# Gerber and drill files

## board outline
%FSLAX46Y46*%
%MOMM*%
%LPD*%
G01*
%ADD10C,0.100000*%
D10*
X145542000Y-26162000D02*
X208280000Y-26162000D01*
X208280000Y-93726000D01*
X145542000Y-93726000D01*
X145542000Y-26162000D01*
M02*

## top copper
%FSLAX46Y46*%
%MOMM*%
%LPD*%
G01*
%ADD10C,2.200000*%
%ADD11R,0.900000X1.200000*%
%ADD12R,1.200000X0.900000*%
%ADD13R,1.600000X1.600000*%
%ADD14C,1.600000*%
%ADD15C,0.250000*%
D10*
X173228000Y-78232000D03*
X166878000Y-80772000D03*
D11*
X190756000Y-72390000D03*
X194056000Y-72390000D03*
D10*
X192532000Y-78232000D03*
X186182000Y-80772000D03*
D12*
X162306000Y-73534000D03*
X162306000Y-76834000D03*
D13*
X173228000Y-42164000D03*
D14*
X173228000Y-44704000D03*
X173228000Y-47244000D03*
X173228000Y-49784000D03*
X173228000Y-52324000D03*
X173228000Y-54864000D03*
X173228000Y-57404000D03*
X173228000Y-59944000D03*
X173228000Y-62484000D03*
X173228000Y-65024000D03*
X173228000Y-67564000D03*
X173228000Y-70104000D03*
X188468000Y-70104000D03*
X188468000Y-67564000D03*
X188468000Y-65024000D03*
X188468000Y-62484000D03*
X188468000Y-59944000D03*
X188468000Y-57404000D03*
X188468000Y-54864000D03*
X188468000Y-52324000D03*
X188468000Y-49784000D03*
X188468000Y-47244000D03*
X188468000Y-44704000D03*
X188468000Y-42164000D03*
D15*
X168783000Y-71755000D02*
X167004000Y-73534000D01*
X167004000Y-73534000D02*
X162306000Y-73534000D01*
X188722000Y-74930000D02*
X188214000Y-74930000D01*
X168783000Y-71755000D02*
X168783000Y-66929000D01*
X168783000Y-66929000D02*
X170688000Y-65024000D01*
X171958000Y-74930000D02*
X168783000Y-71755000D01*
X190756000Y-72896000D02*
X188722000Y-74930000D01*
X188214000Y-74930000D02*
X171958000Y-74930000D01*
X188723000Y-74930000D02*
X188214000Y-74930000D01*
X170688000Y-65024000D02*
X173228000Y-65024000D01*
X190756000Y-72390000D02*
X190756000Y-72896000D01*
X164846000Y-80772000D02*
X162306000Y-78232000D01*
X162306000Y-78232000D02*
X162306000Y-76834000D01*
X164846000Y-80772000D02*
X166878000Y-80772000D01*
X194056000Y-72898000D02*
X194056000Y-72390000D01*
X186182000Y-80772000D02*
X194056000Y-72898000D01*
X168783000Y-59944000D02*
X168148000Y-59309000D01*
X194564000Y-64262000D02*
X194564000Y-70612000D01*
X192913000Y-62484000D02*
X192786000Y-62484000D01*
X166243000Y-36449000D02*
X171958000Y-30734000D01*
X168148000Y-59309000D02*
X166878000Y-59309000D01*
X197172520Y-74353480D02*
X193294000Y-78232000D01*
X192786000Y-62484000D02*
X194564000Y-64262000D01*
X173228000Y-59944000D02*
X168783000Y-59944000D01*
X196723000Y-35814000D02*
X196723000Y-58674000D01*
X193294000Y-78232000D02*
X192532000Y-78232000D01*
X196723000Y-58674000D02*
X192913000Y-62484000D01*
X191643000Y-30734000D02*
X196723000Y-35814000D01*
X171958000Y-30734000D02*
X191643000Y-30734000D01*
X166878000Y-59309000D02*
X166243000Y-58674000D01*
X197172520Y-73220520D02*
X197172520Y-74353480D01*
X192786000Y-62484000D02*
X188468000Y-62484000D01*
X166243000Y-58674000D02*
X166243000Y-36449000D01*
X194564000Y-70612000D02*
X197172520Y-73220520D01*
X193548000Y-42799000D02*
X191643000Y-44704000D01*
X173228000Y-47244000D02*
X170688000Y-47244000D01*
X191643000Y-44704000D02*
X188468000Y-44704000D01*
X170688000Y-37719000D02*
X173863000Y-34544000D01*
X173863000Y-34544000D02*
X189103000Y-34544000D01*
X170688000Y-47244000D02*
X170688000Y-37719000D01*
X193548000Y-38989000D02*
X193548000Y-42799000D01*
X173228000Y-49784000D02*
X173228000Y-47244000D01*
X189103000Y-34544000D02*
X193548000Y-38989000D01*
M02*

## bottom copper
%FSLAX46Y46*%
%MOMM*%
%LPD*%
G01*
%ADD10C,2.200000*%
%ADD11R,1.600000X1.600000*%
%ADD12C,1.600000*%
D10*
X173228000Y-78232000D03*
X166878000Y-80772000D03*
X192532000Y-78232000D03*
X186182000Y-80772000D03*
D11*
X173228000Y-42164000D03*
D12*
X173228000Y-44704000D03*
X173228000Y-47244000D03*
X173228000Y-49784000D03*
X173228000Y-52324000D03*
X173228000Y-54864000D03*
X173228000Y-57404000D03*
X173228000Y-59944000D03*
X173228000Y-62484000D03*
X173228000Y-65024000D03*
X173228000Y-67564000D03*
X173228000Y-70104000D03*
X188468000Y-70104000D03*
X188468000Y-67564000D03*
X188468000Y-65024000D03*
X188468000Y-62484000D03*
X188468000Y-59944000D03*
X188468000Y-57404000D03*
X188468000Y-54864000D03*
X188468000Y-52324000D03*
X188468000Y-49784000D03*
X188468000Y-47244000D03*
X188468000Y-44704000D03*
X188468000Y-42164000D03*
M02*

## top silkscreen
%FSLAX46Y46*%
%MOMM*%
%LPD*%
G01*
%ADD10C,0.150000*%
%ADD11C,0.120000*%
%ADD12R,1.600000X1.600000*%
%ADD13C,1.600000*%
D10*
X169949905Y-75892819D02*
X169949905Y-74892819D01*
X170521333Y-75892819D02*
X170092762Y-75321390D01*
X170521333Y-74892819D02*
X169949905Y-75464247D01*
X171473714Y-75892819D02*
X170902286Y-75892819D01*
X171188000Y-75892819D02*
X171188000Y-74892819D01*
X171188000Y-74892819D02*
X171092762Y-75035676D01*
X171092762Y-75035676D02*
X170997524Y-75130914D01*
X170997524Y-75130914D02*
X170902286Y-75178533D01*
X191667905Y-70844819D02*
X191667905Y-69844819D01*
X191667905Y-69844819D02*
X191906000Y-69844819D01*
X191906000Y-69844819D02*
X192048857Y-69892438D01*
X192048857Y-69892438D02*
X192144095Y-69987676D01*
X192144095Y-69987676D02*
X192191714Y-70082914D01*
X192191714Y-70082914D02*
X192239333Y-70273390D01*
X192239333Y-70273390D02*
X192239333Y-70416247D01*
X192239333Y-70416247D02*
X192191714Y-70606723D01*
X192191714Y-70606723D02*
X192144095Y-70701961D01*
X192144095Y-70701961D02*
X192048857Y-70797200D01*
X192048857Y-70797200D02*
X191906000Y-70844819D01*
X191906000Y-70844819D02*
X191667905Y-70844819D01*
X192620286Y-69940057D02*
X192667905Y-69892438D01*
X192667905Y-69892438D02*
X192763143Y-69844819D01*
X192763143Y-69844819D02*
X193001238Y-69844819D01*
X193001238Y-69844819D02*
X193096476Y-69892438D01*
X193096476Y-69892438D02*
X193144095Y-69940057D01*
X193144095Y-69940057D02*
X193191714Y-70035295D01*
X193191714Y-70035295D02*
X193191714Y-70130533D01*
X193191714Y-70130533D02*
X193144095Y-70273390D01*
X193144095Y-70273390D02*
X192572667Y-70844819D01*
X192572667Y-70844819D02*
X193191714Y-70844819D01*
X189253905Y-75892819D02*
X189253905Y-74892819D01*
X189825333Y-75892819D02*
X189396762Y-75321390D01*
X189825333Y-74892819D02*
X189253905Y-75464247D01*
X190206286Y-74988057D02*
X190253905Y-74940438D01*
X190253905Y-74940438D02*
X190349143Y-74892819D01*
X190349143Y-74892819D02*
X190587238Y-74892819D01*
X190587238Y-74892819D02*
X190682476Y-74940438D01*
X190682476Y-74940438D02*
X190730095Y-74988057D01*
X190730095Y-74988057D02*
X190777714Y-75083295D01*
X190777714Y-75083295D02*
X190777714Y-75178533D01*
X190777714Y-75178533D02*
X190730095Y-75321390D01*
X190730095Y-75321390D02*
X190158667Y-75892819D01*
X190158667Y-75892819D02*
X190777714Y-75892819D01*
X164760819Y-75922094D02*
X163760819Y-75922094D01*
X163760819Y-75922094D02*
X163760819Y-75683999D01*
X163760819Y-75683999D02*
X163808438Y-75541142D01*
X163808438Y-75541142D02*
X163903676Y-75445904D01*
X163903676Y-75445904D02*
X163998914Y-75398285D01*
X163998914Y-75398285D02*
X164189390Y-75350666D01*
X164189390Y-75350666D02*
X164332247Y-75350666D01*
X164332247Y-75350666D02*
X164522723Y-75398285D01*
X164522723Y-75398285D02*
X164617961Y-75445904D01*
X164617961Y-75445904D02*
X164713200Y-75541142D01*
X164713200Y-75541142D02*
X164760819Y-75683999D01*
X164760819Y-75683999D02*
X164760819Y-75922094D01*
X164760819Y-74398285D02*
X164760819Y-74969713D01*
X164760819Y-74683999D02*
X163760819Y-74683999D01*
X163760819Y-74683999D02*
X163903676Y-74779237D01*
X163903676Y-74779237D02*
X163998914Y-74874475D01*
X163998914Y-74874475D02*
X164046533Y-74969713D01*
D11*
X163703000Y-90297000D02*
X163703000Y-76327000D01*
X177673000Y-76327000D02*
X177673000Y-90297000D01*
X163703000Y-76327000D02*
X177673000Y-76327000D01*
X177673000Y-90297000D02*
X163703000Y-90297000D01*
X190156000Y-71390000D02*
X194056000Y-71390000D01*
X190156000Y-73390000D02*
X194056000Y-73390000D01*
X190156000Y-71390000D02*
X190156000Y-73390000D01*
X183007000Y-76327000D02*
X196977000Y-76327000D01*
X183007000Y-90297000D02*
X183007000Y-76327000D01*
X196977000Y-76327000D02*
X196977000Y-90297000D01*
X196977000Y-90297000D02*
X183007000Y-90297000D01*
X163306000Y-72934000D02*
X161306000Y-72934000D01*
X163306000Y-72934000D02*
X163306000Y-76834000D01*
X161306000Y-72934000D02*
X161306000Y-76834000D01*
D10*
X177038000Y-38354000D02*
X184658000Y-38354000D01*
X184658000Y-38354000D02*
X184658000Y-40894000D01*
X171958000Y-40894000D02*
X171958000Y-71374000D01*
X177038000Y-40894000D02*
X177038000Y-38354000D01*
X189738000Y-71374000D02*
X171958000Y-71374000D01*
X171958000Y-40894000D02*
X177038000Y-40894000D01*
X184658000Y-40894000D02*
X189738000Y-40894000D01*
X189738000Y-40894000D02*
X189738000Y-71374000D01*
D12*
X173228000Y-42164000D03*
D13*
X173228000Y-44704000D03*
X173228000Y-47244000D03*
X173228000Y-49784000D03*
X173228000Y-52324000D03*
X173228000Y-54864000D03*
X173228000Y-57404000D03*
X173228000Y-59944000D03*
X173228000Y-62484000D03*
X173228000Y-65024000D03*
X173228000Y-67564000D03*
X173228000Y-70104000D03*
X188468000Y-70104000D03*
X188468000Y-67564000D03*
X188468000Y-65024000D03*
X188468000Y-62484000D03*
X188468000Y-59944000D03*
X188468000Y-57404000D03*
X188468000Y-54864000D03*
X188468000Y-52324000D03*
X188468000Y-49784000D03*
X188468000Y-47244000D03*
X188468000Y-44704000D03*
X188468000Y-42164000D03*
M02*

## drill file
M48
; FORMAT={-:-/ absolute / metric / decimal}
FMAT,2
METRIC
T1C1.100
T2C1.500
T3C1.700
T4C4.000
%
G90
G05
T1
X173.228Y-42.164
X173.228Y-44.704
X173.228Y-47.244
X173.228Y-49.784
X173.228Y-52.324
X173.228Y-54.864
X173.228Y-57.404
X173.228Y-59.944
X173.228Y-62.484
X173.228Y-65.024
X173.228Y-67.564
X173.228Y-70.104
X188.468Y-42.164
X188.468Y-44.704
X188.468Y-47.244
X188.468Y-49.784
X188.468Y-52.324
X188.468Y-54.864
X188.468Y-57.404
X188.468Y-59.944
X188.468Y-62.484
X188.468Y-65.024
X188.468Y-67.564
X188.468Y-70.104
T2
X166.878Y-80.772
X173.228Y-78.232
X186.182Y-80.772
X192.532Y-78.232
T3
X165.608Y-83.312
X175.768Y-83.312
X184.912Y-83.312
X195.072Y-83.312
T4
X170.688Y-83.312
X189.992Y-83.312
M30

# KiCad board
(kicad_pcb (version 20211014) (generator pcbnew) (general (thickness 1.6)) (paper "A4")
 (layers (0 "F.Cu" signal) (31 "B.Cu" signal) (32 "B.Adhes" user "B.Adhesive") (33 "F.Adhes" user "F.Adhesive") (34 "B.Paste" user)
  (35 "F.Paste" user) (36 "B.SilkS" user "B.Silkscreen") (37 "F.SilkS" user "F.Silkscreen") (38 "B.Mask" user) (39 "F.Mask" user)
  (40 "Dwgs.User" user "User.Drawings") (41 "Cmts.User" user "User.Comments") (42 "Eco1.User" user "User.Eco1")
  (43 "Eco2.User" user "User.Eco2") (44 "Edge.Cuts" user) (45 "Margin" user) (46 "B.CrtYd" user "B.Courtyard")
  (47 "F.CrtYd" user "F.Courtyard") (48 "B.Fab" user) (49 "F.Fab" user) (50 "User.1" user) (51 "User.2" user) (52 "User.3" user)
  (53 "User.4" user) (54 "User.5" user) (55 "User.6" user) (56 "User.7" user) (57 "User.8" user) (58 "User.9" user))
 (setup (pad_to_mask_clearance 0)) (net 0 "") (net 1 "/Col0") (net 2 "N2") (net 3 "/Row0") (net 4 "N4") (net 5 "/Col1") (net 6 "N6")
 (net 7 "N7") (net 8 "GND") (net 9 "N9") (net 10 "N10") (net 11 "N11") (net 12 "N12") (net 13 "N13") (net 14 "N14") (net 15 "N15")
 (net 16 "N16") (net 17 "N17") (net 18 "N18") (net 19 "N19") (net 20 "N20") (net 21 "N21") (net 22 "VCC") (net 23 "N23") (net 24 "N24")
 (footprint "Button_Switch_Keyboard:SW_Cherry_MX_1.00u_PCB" (layer "F.Cu") (at 173.228 78.232)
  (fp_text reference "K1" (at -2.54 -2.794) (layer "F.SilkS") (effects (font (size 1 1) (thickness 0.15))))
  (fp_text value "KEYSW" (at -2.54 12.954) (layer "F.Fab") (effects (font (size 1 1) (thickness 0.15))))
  (fp_line (start -9.525 12.065) (end -9.525 -1.905) (layer "F.SilkS") (width 0.12))
  (fp_line (start 4.445 -1.905) (end 4.445 12.065) (layer "F.SilkS") (width 0.12))
  (fp_line (start -9.525 -1.905) (end 4.445 -1.905) (layer "F.SilkS") (width 0.12))
  (fp_line (start 4.445 12.065) (end -9.525 12.065) (layer "F.SilkS") (width 0.12))
  (pad "" np_thru_hole circle (at 2.54 5.08) (size 1.7 1.7) (drill 1.7) (layers *.Cu *.Mask))
  (pad "" np_thru_hole circle (at -7.62 5.08) (size 1.7 1.7) (drill 1.7) (layers *.Cu *.Mask))
  (pad "" np_thru_hole circle (at -2.54 5.08) (size 4 4) (drill 4) (layers *.Cu *.Mask))
  (pad "1" thru_hole circle (at 0 0) (size 2.2 2.2) (drill 1.5) (layers *.Cu *.Mask) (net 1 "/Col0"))
  (pad "2" thru_hole circle (at -6.35 2.54) (size 2.2 2.2) (drill 1.5) (layers *.Cu *.Mask) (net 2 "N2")))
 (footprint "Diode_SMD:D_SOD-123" (layer "F.Cu") (at 192.406 72.39)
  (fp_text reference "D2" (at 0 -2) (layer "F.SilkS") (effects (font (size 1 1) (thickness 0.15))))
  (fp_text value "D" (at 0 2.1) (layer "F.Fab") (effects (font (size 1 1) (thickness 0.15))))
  (fp_line (start -2.25 -1) (end 1.65 -1) (layer "F.SilkS") (width 0.12))
  (fp_line (start -2.25 1) (end 1.65 1) (layer "F.SilkS") (width 0.12))
  (fp_line (start -2.25 -1) (end -2.25 1) (layer "F.SilkS") (width 0.12))
  (pad "1" smd rect (at -1.65 0) (size 0.9 1.2) (layers "F.Cu" "F.Paste" "F.Mask") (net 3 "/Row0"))
  (pad "2" smd rect (at 1.65 0) (size 0.9 1.2) (layers "F.Cu" "F.Paste" "F.Mask") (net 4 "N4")))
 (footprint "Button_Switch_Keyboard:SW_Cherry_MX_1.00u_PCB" (layer "F.Cu") (at 192.532 78.232)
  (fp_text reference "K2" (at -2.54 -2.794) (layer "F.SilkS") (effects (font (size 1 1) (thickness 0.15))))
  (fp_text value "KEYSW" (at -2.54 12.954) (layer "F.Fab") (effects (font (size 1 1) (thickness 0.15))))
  (fp_line (start -9.525 -1.905) (end 4.445 -1.905) (layer "F.SilkS") (width 0.12))
  (fp_line (start -9.525 12.065) (end -9.525 -1.905) (layer "F.SilkS") (width 0.12))
  (fp_line (start 4.445 -1.905) (end 4.445 12.065) (layer "F.SilkS") (width 0.12))
  (fp_line (start 4.445 12.065) (end -9.525 12.065) (layer "F.SilkS") (width 0.12))
  (pad "" np_thru_hole circle (at -2.54 5.08) (size 4 4) (drill 4) (layers *.Cu *.Mask))
  (pad "" np_thru_hole circle (at 2.54 5.08) (size 1.7 1.7) (drill 1.7) (layers *.Cu *.Mask))
  (pad "" np_thru_hole circle (at -7.62 5.08) (size 1.7 1.7) (drill 1.7) (layers *.Cu *.Mask))
  (pad "1" thru_hole circle (at 0 0) (size 2.2 2.2) (drill 1.5) (layers *.Cu *.Mask) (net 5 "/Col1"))
  (pad "2" thru_hole circle (at -6.35 2.54) (size 2.2 2.2) (drill 1.5) (layers *.Cu *.Mask) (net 4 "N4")))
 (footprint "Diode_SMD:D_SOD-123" (layer "F.Cu") (at 162.306 75.184 -90)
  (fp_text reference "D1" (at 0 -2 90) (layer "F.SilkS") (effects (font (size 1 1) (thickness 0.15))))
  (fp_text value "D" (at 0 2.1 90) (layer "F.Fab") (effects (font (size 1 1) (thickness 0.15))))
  (fp_line (start -2.25 -1) (end -2.25 1) (layer "F.SilkS") (width 0.12))
  (fp_line (start -2.25 -1) (end 1.65 -1) (layer "F.SilkS") (width 0.12))
  (fp_line (start -2.25 1) (end 1.65 1) (layer "F.SilkS") (width 0.12))
  (pad "1" smd rect (at -1.65 0 270) (size 0.9 1.2) (layers "F.Cu" "F.Paste" "F.Mask") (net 3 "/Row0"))
  (pad "2" smd rect (at 1.65 0 270) (size 0.9 1.2) (layers "F.Cu" "F.Paste" "F.Mask") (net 2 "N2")))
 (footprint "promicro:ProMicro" (layer "F.Cu") (at 180.848 56.134 -90)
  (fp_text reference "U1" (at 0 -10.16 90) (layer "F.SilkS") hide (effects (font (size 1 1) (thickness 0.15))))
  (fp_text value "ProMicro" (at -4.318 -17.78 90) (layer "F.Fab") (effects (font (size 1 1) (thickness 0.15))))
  (fp_line (start -17.78 3.81) (end -17.78 -3.81) (layer "F.SilkS") (width 0.15))
  (fp_line (start -17.78 -3.81) (end -15.24 -3.81) (layer "F.SilkS") (width 0.15))
  (fp_line (start -15.24 8.89) (end 15.24 8.89) (layer "F.SilkS") (width 0.15))
  (fp_line (start -15.24 3.81) (end -17.78 3.81) (layer "F.SilkS") (width 0.15))
  (fp_line (start 15.24 -8.89) (end 15.24 8.89) (layer "F.SilkS") (width 0.15))
  (fp_line (start -15.24 8.89) (end -15.24 3.81) (layer "F.SilkS") (width 0.15))
  (fp_line (start -15.24 -3.81) (end -15.24 -8.89) (layer "F.SilkS") (width 0.15))
  (fp_line (start -15.24 -8.89) (end 15.24 -8.89) (layer "F.SilkS") (width 0.15))
  (pad "1" thru_hole rect locked (at -13.97 7.62 270) (size 1.6 1.6) (drill 1.1) (layers *.Cu *.Mask "F.SilkS") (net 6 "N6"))
  (pad "2" thru_hole circle locked (at -11.43 7.62 270) (size 1.6 1.6) (drill 1.1) (layers *.Cu *.Mask "F.SilkS") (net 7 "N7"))
  (pad "3" thru_hole circle locked (at -8.89 7.62 270) (size 1.6 1.6) (drill 1.1) (layers *.Cu *.Mask "F.SilkS") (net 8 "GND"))
  (pad "4" thru_hole circle locked (at -6.35 7.62 270) (size 1.6 1.6) (drill 1.1) (layers *.Cu *.Mask "F.SilkS") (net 8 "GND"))
  (pad "5" thru_hole circle locked (at -3.81 7.62 270) (size 1.6 1.6) (drill 1.1) (layers *.Cu *.Mask "F.SilkS") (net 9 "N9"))
  (pad "6" thru_hole circle locked (at -1.27 7.62 270) (size 1.6 1.6) (drill 1.1) (layers *.Cu *.Mask "F.SilkS") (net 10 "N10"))
  (pad "7" thru_hole circle locked (at 1.27 7.62 270) (size 1.6 1.6) (drill 1.1) (layers *.Cu *.Mask "F.SilkS") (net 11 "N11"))
  (pad "8" thru_hole circle locked (at 3.81 7.62 270) (size 1.6 1.6) (drill 1.1) (layers *.Cu *.Mask "F.SilkS") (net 5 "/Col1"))
  (pad "9" thru_hole circle locked (at 6.35 7.62 270) (size 1.6 1.6) (drill 1.1) (layers *.Cu *.Mask "F.SilkS") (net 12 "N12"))
  (pad "10" thru_hole circle locked (at 8.89 7.62 270) (size 1.6 1.6) (drill 1.1) (layers *.Cu *.Mask "F.SilkS") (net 3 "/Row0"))
  (pad "11" thru_hole circle locked (at 11.43 7.62 270) (size 1.6 1.6) (drill 1.1) (layers *.Cu *.Mask "F.SilkS") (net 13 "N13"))
  (pad "12" thru_hole circle locked (at 13.97 7.62 270) (size 1.6 1.6) (drill 1.1) (layers *.Cu *.Mask "F.SilkS") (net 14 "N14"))
  (pad "13" thru_hole circle locked (at 13.97 -7.62 270) (size 1.6 1.6) (drill 1.1) (layers *.Cu *.Mask "F.SilkS") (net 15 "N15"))
  (pad "14" thru_hole circle locked (at 11.43 -7.62 270) (size 1.6 1.6) (drill 1.1) (layers *.Cu *.Mask "F.SilkS") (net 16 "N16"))
  (pad "15" thru_hole circle locked (at 8.89 -7.62 270) (size 1.6 1.6) (drill 1.1) (layers *.Cu *.Mask "F.SilkS") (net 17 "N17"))
  (pad "16" thru_hole circle locked (at 6.35 -7.62 270) (size 1.6 1.6) (drill 1.1) (layers *.Cu *.Mask "F.SilkS") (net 5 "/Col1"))
  (pad "17" thru_hole circle locked (at 3.81 -7.62 270) (size 1.6 1.6) (drill 1.1) (layers *.Cu *.Mask "F.SilkS") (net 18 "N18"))
  (pad "18" thru_hole circle locked (at 1.27 -7.62 270) (size 1.6 1.6) (drill 1.1) (layers *.Cu *.Mask "F.SilkS") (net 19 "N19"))
  (pad "19" thru_hole circle locked (at -1.27 -7.62 270) (size 1.6 1.6) (drill 1.1) (layers *.Cu *.Mask "F.SilkS") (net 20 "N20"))
  (pad "20" thru_hole circle locked (at -3.81 -7.62 270) (size 1.6 1.6) (drill 1.1) (layers *.Cu *.Mask "F.SilkS") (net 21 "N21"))
  (pad "21" thru_hole circle locked (at -6.35 -7.62 270) (size 1.6 1.6) (drill 1.1) (layers *.Cu *.Mask "F.SilkS") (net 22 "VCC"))
  (pad "22" thru_hole circle locked (at -8.89 -7.62 270) (size 1.6 1.6) (drill 1.1) (layers *.Cu *.Mask "F.SilkS") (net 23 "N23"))
  (pad "23" thru_hole circle locked (at -11.43 -7.62 270) (size 1.6 1.6) (drill 1.1) (layers *.Cu *.Mask "F.SilkS") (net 8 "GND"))
  (pad "24" thru_hole circle locked (at -13.97 -7.62 270) (size 1.6 1.6) (drill 1.1) (layers *.Cu *.Mask "F.SilkS") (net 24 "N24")))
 (gr_rect (start 145.542 26.162) (end 208.28 93.726) (layer "Edge.Cuts") (width 0.1) (fill none))
 (segment (start 168.783 71.755) (end 167.004 73.534) (width 0.25) (layer "F.Cu") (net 3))
 (segment (start 167.004 73.534) (end 162.306 73.534) (width 0.25) (layer "F.Cu") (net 3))
 (segment (start 188.722 74.93) (end 188.214 74.93) (width 0.25) (layer "F.Cu") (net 3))
 (segment (start 168.783 71.755) (end 168.783 66.929) (width 0.25) (layer "F.Cu") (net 3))
 (segment (start 168.783 66.929) (end 170.688 65.024) (width 0.25) (layer "F.Cu") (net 3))
 (segment (start 171.958 74.93) (end 168.783 71.755) (width 0.25) (layer "F.Cu") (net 3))
 (segment (start 190.756 72.896) (end 188.722 74.93) (width 0.25) (layer "F.Cu") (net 3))
 (segment (start 188.214 74.93) (end 171.958 74.93) (width 0.25) (layer "F.Cu") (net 3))
 (segment (start 188.723 74.93) (end 188.214 74.93) (width 0.25) (layer "F.Cu") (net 3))
 (segment (start 170.688 65.024) (end 173.228 65.024) (width 0.25) (layer "F.Cu") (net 3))
 (segment (start 190.756 72.39) (end 190.756 72.896) (width 0.25) (layer "F.Cu") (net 3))
 (segment (start 164.846 80.772) (end 162.306 78.232) (width 0.25) (layer "F.Cu") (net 2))
 (segment (start 162.306 78.232) (end 162.306 76.834) (width 0.25) (layer "F.Cu") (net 2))
 (segment (start 164.846 80.772) (end 166.878 80.772) (width 0.25) (layer "F.Cu") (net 2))
 (segment (start 194.056 72.898) (end 194.056 72.39) (width 0.25) (layer "F.Cu") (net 4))
 (segment (start 186.182 80.772) (end 194.056 72.898) (width 0.25) (layer "F.Cu") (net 4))
 (segment (start 168.783 59.944) (end 168.148 59.309) (width 0.25) (layer "F.Cu") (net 5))
 (segment (start 194.564 64.262) (end 194.564 70.612) (width 0.25) (layer "F.Cu") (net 5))
 (segment (start 192.913 62.484) (end 192.786 62.484) (width 0.25) (layer "F.Cu") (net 5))
 (segment (start 166.243 36.449) (end 171.958 30.734) (width 0.25) (layer "F.Cu") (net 5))
 (segment (start 168.148 59.309) (end 166.878 59.309) (width 0.25) (layer "F.Cu") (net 5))
 (segment (start 197.17252 74.35348) (end 193.294 78.232) (width 0.25) (layer "F.Cu") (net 5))
 (segment (start 192.786 62.484) (end 194.564 64.262) (width 0.25) (layer "F.Cu") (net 5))
 (segment (start 173.228 59.944) (end 168.783 59.944) (width 0.25) (layer "F.Cu") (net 5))
 (segment (start 196.723 35.814) (end 196.723 58.674) (width 0.25) (layer "F.Cu") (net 5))
 (segment (start 193.294 78.232) (end 192.532 78.232) (width 0.25) (layer "F.Cu") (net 5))
 (segment (start 196.723 58.674) (end 192.913 62.484) (width 0.25) (layer "F.Cu") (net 5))
 (segment (start 191.643 30.734) (end 196.723 35.814) (width 0.25) (layer "F.Cu") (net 5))
 (segment (start 171.958 30.734) (end 191.643 30.734) (width 0.25) (layer "F.Cu") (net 5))
 (segment (start 166.878 59.309) (end 166.243 58.674) (width 0.25) (layer "F.Cu") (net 5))
 (segment (start 197.17252 73.22052) (end 197.17252 74.35348) (width 0.25) (layer "F.Cu") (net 5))
 (segment (start 192.786 62.484) (end 188.468 62.484) (width 0.25) (layer "F.Cu") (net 5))
 (segment (start 166.243 58.674) (end 166.243 36.449) (width 0.25) (layer "F.Cu") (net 5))
 (segment (start 194.564 70.612) (end 197.17252 73.22052) (width 0.25) (layer "F.Cu") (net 5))
 (segment (start 193.548 42.799) (end 191.643 44.704) (width 0.25) (layer "F.Cu") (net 8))
 (segment (start 173.228 47.244) (end 170.688 47.244) (width 0.25) (layer "F.Cu") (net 8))
 (segment (start 191.643 44.704) (end 188.468 44.704) (width 0.25) (layer "F.Cu") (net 8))
 (segment (start 170.688 37.719) (end 173.863 34.544) (width 0.25) (layer "F.Cu") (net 8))
 (segment (start 173.863 34.544) (end 189.103 34.544) (width 0.25) (layer "F.Cu") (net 8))
 (segment (start 170.688 47.244) (end 170.688 37.719) (width 0.25) (layer "F.Cu") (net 8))
 (segment (start 193.548 38.989) (end 193.548 42.799) (width 0.25) (layer "F.Cu") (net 8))
 (segment (start 173.228 49.784) (end 173.228 47.244) (width 0.25) (layer "F.Cu") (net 8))
 (segment (start 189.103 34.544) (end 193.548 38.989) (width 0.25) (layer "F.Cu") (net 8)))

